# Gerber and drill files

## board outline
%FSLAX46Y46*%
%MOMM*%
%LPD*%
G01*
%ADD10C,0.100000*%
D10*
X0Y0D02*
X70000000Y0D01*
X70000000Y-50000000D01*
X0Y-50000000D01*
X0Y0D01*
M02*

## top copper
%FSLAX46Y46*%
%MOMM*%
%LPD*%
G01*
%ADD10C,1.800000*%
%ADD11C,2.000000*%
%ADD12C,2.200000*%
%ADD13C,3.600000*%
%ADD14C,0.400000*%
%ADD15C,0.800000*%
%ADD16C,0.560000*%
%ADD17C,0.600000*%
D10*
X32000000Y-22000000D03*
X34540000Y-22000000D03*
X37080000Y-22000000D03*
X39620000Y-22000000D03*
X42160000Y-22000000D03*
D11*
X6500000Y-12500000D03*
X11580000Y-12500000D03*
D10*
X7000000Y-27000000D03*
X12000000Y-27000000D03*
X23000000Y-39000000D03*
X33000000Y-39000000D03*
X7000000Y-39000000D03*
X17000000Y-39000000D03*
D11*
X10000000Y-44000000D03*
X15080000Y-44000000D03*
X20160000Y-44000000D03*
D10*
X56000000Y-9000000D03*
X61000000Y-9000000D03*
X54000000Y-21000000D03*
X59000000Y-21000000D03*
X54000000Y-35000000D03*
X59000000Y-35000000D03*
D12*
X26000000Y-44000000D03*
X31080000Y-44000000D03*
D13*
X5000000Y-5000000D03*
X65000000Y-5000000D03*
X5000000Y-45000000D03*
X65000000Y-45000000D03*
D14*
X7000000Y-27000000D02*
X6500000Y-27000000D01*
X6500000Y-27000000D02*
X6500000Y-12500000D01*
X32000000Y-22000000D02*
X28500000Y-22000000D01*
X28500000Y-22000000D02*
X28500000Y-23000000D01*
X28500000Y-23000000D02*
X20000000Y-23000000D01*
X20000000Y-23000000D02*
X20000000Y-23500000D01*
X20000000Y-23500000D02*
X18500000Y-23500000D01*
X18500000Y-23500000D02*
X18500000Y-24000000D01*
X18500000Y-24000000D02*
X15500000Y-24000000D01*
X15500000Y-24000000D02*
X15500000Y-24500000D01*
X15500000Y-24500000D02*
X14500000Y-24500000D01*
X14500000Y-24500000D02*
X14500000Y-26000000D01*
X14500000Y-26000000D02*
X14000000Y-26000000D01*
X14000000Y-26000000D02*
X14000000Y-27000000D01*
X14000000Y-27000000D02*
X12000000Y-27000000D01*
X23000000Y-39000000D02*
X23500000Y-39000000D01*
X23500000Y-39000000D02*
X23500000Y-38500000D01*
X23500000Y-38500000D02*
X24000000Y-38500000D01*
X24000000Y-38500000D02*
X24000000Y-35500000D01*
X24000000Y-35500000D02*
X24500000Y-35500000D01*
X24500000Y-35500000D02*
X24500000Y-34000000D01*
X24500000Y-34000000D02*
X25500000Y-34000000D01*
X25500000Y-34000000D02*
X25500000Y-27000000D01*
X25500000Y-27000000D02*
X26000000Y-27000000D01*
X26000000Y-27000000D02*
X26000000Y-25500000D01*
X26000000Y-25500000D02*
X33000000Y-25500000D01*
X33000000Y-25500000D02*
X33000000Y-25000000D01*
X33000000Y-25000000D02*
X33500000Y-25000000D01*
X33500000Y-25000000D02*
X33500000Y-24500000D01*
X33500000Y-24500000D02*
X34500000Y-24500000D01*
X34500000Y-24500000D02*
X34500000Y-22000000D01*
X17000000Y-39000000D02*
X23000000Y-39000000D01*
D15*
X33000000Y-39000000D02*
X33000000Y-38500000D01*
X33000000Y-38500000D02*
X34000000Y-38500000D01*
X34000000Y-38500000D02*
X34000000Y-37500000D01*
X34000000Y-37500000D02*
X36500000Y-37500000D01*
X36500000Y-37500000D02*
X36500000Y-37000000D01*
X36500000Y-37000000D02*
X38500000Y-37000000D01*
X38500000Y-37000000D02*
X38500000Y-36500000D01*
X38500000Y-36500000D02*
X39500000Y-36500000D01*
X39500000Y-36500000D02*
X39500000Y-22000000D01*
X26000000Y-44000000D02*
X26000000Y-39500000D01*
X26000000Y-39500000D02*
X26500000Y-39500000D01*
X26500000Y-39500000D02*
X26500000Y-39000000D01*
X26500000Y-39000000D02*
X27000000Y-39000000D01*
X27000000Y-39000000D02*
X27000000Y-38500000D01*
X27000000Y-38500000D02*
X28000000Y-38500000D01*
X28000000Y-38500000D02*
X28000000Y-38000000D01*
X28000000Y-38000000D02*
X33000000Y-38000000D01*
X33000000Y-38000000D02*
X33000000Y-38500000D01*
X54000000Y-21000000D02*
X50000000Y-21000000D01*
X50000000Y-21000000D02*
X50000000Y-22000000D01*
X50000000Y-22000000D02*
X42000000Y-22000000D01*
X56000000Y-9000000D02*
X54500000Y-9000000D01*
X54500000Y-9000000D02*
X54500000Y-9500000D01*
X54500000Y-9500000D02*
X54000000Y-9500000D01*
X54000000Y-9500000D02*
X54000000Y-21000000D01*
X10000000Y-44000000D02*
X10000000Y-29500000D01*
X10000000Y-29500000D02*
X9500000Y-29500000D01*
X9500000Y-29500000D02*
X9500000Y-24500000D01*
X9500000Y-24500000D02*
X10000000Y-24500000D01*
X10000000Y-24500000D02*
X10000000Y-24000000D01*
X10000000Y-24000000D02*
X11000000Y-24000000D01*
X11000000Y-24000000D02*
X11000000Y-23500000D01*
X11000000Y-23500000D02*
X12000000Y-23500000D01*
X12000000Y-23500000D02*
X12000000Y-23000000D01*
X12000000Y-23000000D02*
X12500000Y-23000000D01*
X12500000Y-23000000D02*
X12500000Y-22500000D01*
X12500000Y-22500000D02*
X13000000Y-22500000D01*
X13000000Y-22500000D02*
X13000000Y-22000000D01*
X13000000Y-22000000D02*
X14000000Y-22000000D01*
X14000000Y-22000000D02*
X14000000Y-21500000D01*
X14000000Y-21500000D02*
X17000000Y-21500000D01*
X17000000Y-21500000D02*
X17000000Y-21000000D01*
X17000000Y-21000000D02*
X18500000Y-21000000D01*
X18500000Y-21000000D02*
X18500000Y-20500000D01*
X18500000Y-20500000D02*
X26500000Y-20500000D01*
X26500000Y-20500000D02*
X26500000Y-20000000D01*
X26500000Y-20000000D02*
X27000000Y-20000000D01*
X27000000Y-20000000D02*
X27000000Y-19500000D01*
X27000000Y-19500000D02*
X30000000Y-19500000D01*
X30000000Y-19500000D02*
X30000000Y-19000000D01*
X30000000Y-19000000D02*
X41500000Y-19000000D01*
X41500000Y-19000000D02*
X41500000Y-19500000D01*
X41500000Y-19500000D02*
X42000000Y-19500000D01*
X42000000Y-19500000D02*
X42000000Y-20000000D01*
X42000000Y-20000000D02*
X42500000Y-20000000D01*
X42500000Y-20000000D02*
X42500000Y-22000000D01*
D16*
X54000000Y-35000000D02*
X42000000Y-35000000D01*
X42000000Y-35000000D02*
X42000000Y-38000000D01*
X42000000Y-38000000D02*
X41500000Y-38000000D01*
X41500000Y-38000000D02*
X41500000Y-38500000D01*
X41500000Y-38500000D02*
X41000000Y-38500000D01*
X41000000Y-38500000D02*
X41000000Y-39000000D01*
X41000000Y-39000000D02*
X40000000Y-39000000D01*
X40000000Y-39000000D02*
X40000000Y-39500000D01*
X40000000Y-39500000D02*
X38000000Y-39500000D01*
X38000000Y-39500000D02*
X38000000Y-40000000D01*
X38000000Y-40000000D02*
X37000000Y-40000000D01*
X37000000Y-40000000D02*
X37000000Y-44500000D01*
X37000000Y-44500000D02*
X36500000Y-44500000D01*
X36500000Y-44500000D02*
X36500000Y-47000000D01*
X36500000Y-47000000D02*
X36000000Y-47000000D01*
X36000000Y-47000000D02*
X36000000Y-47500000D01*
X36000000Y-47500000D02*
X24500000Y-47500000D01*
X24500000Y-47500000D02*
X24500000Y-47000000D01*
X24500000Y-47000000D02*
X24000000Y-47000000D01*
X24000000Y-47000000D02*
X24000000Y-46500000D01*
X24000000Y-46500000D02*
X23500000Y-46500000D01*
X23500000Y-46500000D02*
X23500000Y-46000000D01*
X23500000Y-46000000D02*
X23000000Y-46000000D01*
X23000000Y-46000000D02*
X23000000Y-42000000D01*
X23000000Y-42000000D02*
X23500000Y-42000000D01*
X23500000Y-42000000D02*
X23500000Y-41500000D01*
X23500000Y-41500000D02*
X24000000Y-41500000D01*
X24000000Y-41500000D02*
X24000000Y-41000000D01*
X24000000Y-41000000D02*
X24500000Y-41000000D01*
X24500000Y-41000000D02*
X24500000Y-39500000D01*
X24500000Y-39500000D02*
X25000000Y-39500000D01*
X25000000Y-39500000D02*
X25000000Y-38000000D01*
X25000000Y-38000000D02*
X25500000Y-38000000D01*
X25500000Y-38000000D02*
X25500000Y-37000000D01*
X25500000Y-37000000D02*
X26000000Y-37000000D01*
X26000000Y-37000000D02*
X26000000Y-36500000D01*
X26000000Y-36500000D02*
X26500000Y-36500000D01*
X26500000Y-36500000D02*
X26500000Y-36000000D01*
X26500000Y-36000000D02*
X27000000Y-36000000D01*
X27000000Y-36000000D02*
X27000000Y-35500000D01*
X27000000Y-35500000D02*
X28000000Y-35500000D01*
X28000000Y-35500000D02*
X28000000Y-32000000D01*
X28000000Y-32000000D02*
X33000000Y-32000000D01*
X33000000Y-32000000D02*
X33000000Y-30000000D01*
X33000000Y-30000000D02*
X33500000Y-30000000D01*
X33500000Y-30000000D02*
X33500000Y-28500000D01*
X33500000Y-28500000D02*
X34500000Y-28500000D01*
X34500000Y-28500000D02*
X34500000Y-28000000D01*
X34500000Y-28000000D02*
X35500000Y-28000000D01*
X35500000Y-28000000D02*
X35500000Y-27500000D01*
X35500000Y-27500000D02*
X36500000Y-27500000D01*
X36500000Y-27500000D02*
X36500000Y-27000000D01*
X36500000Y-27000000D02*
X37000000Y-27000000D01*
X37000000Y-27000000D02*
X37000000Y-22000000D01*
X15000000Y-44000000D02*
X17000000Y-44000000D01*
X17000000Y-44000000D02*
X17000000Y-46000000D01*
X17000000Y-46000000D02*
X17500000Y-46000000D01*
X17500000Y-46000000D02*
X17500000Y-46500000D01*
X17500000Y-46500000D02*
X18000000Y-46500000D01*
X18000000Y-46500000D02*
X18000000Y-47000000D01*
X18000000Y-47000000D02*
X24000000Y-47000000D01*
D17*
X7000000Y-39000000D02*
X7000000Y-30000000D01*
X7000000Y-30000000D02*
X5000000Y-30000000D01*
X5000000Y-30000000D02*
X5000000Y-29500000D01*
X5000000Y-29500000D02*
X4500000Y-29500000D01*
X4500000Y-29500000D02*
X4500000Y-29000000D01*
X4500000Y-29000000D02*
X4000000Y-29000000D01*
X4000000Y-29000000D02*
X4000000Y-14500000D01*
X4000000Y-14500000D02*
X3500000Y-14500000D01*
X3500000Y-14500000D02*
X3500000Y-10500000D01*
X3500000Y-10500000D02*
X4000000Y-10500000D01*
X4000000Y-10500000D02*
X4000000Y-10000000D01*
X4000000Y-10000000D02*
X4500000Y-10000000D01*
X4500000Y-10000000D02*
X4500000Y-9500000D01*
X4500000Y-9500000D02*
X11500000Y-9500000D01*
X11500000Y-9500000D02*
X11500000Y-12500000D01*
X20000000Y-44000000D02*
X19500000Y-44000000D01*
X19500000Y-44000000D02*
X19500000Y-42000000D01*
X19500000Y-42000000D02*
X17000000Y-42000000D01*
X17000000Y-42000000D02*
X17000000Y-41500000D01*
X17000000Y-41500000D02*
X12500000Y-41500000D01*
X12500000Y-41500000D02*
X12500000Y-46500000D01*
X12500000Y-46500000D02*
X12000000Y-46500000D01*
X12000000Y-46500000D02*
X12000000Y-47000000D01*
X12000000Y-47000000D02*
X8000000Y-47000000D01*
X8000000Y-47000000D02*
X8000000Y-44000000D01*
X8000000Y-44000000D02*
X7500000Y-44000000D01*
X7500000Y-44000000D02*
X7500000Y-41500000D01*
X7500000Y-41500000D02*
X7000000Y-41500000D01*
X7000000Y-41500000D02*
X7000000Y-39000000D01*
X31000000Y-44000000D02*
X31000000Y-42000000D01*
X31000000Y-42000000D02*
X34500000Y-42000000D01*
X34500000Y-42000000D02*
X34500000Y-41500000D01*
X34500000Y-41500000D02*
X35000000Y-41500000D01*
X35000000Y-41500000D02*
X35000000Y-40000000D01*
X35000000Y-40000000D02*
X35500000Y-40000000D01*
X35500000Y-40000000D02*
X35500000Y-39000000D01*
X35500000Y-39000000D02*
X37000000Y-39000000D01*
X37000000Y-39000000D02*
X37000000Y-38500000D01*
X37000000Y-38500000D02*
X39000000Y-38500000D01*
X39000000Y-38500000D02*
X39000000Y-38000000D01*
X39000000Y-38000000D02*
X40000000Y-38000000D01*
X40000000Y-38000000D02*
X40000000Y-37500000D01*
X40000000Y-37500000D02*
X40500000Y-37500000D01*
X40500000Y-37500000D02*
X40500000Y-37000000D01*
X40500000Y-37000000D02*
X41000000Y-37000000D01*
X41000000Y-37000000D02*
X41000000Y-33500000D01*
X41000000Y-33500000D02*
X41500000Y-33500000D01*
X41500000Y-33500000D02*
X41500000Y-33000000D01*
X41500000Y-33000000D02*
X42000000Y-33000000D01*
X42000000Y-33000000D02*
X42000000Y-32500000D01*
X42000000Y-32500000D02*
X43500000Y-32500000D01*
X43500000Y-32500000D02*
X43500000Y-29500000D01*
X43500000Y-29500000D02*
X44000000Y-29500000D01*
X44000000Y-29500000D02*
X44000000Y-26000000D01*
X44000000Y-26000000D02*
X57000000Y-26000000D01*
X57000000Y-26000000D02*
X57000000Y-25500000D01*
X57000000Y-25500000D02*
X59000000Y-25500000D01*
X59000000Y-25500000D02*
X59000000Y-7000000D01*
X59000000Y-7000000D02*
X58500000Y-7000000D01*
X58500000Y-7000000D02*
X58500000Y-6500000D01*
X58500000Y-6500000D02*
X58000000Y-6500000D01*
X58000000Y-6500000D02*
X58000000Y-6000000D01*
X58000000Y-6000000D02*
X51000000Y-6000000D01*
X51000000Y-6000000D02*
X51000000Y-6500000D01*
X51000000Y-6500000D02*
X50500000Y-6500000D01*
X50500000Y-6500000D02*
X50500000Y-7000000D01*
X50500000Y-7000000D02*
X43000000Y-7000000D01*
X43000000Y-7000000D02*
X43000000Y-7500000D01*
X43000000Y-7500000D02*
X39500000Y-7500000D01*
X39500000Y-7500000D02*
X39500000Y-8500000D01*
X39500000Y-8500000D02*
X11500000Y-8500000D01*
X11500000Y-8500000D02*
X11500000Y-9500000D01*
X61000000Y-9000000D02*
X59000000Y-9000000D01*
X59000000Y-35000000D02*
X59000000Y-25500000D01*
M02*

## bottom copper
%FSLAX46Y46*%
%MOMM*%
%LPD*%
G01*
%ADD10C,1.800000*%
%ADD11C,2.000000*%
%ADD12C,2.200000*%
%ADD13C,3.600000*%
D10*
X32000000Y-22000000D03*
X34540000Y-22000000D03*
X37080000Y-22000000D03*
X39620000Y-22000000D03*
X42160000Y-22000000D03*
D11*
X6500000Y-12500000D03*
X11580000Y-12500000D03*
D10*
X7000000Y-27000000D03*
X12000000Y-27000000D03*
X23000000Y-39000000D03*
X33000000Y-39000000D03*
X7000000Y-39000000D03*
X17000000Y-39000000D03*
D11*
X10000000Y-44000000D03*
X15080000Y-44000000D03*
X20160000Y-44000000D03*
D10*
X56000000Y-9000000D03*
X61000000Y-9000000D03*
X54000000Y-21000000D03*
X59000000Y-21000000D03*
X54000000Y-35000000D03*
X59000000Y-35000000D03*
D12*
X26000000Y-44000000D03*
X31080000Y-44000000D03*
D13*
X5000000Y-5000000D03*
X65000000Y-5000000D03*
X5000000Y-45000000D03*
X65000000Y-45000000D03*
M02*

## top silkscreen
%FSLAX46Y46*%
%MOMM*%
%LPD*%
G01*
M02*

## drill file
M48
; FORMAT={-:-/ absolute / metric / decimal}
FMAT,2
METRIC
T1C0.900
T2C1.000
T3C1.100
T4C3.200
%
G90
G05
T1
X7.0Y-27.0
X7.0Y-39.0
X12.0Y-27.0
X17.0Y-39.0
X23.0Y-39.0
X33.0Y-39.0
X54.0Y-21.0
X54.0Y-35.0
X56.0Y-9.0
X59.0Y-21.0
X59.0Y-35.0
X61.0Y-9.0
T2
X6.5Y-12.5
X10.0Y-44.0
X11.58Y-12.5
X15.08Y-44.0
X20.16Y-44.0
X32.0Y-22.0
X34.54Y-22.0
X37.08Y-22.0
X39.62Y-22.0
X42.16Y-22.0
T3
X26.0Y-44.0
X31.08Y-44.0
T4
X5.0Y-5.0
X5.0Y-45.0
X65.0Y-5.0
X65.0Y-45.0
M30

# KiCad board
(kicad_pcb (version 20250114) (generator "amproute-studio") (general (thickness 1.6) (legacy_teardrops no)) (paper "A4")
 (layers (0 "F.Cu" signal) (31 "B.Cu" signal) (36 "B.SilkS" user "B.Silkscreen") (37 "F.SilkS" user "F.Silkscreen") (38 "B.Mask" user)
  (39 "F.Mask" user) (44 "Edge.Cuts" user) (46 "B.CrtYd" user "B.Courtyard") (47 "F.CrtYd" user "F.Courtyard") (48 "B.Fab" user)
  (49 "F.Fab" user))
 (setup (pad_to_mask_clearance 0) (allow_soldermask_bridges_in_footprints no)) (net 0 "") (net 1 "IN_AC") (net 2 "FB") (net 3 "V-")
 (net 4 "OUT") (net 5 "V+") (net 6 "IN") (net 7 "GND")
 (gr_rect (start 0 0) (end 70.0000 50.0000) (stroke (width 0.1) (type default)) (fill none) (layer "Edge.Cuts"))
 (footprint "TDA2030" (layer "F.Cu") (at 30.0000 14.0000)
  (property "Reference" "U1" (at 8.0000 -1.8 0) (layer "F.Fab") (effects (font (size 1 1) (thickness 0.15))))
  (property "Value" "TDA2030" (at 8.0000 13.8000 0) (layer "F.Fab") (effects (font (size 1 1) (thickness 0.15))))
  (pad "1" thru_hole circle (at 2.0000 8.0000) (size 1.8000 1.8000) (drill 1.0000) (layers "*.Cu" "*.Mask") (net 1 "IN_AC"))
  (pad "2" thru_hole circle (at 4.5400 8.0000) (size 1.8000 1.8000) (drill 1.0000) (layers "*.Cu" "*.Mask") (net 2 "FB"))
  (pad "3" thru_hole circle (at 7.0800 8.0000) (size 1.8000 1.8000) (drill 1.0000) (layers "*.Cu" "*.Mask") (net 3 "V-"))
  (pad "4" thru_hole circle (at 9.6200 8.0000) (size 1.8000 1.8000) (drill 1.0000) (layers "*.Cu" "*.Mask") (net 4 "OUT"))
  (pad "5" thru_hole circle (at 12.1600 8.0000) (size 1.8000 1.8000) (drill 1.0000) (layers "*.Cu" "*.Mask") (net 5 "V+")))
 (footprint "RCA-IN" (layer "F.Cu") (at 4.0000 8.0000)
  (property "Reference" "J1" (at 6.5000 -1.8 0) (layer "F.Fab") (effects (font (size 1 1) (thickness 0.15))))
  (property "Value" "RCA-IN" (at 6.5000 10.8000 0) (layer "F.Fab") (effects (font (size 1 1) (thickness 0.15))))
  (pad "1" thru_hole circle (at 2.5000 4.5000) (size 2.0000 2.0000) (drill 1.0000) (layers "*.Cu" "*.Mask") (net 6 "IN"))
  (pad "2" thru_hole circle (at 7.5800 4.5000) (size 2.0000 2.0000) (drill 1.0000) (layers "*.Cu" "*.Mask") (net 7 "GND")))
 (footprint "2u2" (layer "F.Cu") (at 5.0000 24.0000)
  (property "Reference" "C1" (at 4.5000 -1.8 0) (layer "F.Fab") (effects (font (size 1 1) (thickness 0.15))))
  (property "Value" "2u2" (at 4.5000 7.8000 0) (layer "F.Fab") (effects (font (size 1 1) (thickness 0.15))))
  (pad "1" thru_hole circle (at 2.0000 3.0000) (size 1.8000 1.8000) (drill 0.9000) (layers "*.Cu" "*.Mask") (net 6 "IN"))
  (pad "2" thru_hole circle (at 7.0000 3.0000) (size 1.8000 1.8000) (drill 0.9000) (layers "*.Cu" "*.Mask") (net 1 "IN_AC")))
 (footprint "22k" (layer "F.Cu") (at 22.0000 36.0000)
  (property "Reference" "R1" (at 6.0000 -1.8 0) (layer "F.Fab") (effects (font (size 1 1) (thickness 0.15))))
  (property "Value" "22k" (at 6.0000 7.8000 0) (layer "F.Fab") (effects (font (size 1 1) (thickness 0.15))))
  (pad "1" thru_hole circle (at 1.0000 3.0000) (size 1.8000 1.8000) (drill 0.9000) (layers "*.Cu" "*.Mask") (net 2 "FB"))
  (pad "2" thru_hole circle (at 11.0000 3.0000) (size 1.8000 1.8000) (drill 0.9000) (layers "*.Cu" "*.Mask") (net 4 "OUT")))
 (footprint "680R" (layer "F.Cu") (at 6.0000 36.0000)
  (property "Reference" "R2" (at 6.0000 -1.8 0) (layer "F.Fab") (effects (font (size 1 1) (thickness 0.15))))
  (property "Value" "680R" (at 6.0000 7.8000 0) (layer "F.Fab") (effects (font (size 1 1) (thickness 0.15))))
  (pad "1" thru_hole circle (at 1.0000 3.0000) (size 1.8000 1.8000) (drill 0.9000) (layers "*.Cu" "*.Mask") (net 7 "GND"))
  (pad "2" thru_hole circle (at 11.0000 3.0000) (size 1.8000 1.8000) (drill 0.9000) (layers "*.Cu" "*.Mask") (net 2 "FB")))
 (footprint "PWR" (layer "F.Cu") (at 8.0000 40.0000)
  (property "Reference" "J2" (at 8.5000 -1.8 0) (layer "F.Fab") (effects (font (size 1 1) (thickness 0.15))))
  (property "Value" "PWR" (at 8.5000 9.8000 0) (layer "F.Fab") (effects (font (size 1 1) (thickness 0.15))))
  (pad "1" thru_hole circle (at 2.0000 4.0000) (size 2.0000 2.0000) (drill 1.0000) (layers "*.Cu" "*.Mask") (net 5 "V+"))
  (pad "2" thru_hole circle (at 7.0800 4.0000) (size 2.0000 2.0000) (drill 1.0000) (layers "*.Cu" "*.Mask") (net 3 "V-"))
  (pad "3" thru_hole circle (at 12.1600 4.0000) (size 2.0000 2.0000) (drill 1.0000) (layers "*.Cu" "*.Mask") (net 7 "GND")))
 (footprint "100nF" (layer "F.Cu") (at 54.0000 6.0000)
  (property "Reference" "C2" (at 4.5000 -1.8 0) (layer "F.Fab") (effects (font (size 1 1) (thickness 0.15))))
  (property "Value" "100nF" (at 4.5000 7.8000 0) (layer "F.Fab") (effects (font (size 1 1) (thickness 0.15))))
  (pad "1" thru_hole circle (at 2.0000 3.0000) (size 1.8000 1.8000) (drill 0.9000) (layers "*.Cu" "*.Mask") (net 5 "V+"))
  (pad "2" thru_hole circle (at 7.0000 3.0000) (size 1.8000 1.8000) (drill 0.9000) (layers "*.Cu" "*.Mask") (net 7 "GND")))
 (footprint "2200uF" (layer "F.Cu") (at 52.0000 18.0000)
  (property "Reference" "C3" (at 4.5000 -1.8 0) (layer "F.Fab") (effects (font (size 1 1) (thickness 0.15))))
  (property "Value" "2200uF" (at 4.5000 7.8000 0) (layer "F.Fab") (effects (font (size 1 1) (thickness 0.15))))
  (pad "1" thru_hole circle (at 2.0000 3.0000) (size 1.8000 1.8000) (drill 0.9000) (layers "*.Cu" "*.Mask") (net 5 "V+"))
  (pad "2" thru_hole circle (at 7.0000 3.0000) (size 1.8000 1.8000) (drill 0.9000) (layers "*.Cu" "*.Mask") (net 7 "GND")))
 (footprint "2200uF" (layer "F.Cu") (at 52.0000 32.0000)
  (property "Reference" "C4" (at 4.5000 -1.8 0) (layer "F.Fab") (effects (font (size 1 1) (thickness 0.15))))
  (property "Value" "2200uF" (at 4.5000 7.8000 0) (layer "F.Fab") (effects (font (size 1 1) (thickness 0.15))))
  (pad "1" thru_hole circle (at 2.0000 3.0000) (size 1.8000 1.8000) (drill 0.9000) (layers "*.Cu" "*.Mask") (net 3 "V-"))
  (pad "2" thru_hole circle (at 7.0000 3.0000) (size 1.8000 1.8000) (drill 0.9000) (layers "*.Cu" "*.Mask") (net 7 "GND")))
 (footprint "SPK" (layer "F.Cu") (at 24.0000 40.0000)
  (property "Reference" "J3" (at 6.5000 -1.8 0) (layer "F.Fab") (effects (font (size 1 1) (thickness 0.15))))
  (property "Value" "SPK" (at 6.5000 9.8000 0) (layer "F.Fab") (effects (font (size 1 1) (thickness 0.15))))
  (pad "1" thru_hole circle (at 2.0000 4.0000) (size 2.2000 2.2000) (drill 1.1000) (layers "*.Cu" "*.Mask") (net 4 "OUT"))
  (pad "2" thru_hole circle (at 7.0800 4.0000) (size 2.2000 2.2000) (drill 1.1000) (layers "*.Cu" "*.Mask") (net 7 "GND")))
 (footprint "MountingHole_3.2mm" (layer "F.Cu") (at 5.0000 5.0000)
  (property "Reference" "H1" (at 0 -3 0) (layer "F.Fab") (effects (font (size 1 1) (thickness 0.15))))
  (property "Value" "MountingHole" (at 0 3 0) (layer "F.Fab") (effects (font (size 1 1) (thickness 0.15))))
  (pad "" np_thru_hole circle (at 0 0) (size 3.6000 3.6000) (drill 3.2000) (layers "*.Cu" "*.Mask")))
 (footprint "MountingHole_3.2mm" (layer "F.Cu") (at 65.0000 5.0000)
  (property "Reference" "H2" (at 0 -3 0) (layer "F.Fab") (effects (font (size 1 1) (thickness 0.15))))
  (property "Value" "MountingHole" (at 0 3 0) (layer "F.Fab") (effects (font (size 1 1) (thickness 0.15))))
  (pad "" np_thru_hole circle (at 0 0) (size 3.6000 3.6000) (drill 3.2000) (layers "*.Cu" "*.Mask")))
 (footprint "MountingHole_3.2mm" (layer "F.Cu") (at 5.0000 45.0000)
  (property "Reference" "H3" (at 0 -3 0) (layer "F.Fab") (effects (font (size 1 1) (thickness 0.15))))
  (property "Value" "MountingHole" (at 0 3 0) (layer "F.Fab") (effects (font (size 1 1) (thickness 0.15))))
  (pad "" np_thru_hole circle (at 0 0) (size 3.6000 3.6000) (drill 3.2000) (layers "*.Cu" "*.Mask")))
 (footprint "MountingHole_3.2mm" (layer "F.Cu") (at 65.0000 45.0000)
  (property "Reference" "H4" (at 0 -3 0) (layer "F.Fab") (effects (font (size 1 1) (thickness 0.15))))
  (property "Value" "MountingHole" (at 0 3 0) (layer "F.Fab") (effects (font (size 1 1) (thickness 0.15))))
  (pad "" np_thru_hole circle (at 0 0) (size 3.6000 3.6000) (drill 3.2000) (layers "*.Cu" "*.Mask")))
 (segment (start 7.0000 27.0000) (end 6.5000 27.0000) (width 0.4000) (layer "F.Cu") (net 6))
 (segment (start 6.5000 27.0000) (end 6.5000 12.5000) (width 0.4000) (layer "F.Cu") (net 6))
 (segment (start 32.0000 22.0000) (end 28.5000 22.0000) (width 0.4000) (layer "F.Cu") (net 1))
 (segment (start 28.5000 22.0000) (end 28.5000 23.0000) (width 0.4000) (layer "F.Cu") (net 1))
 (segment (start 28.5000 23.0000) (end 20.0000 23.0000) (width 0.4000) (layer "F.Cu") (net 1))
 (segment (start 20.0000 23.0000) (end 20.0000 23.5000) (width 0.4000) (layer "F.Cu") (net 1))
 (segment (start 20.0000 23.5000) (end 18.5000 23.5000) (width 0.4000) (layer "F.Cu") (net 1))
 (segment (start 18.5000 23.5000) (end 18.5000 24.0000) (width 0.4000) (layer "F.Cu") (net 1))
 (segment (start 18.5000 24.0000) (end 15.5000 24.0000) (width 0.4000) (layer "F.Cu") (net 1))
 (segment (start 15.5000 24.0000) (end 15.5000 24.5000) (width 0.4000) (layer "F.Cu") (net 1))
 (segment (start 15.5000 24.5000) (end 14.5000 24.5000) (width 0.4000) (layer "F.Cu") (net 1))
 (segment (start 14.5000 24.5000) (end 14.5000 26.0000) (width 0.4000) (layer "F.Cu") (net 1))
 (segment (start 14.5000 26.0000) (end 14.0000 26.0000) (width 0.4000) (layer "F.Cu") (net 1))
 (segment (start 14.0000 26.0000) (end 14.0000 27.0000) (width 0.4000) (layer "F.Cu") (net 1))
 (segment (start 14.0000 27.0000) (end 12.0000 27.0000) (width 0.4000) (layer "F.Cu") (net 1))
 (segment (start 23.0000 39.0000) (end 23.5000 39.0000) (width 0.4000) (layer "F.Cu") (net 2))
 (segment (start 23.5000 39.0000) (end 23.5000 38.5000) (width 0.4000) (layer "F.Cu") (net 2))
 (segment (start 23.5000 38.5000) (end 24.0000 38.5000) (width 0.4000) (layer "F.Cu") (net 2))
 (segment (start 24.0000 38.5000) (end 24.0000 35.5000) (width 0.4000) (layer "F.Cu") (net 2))
 (segment (start 24.0000 35.5000) (end 24.5000 35.5000) (width 0.4000) (layer "F.Cu") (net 2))
 (segment (start 24.5000 35.5000) (end 24.5000 34.0000) (width 0.4000) (layer "F.Cu") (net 2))
 (segment (start 24.5000 34.0000) (end 25.5000 34.0000) (width 0.4000) (layer "F.Cu") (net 2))
 (segment (start 25.5000 34.0000) (end 25.5000 27.0000) (width 0.4000) (layer "F.Cu") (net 2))
 (segment (start 25.5000 27.0000) (end 26.0000 27.0000) (width 0.4000) (layer "F.Cu") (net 2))
 (segment (start 26.0000 27.0000) (end 26.0000 25.5000) (width 0.4000) (layer "F.Cu") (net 2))
 (segment (start 26.0000 25.5000) (end 33.0000 25.5000) (width 0.4000) (layer "F.Cu") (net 2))
 (segment (start 33.0000 25.5000) (end 33.0000 25.0000) (width 0.4000) (layer "F.Cu") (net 2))
 (segment (start 33.0000 25.0000) (end 33.5000 25.0000) (width 0.4000) (layer "F.Cu") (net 2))
 (segment (start 33.5000 25.0000) (end 33.5000 24.5000) (width 0.4000) (layer "F.Cu") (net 2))
 (segment (start 33.5000 24.5000) (end 34.5000 24.5000) (width 0.4000) (layer "F.Cu") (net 2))
 (segment (start 34.5000 24.5000) (end 34.5000 22.0000) (width 0.4000) (layer "F.Cu") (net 2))
 (segment (start 17.0000 39.0000) (end 23.0000 39.0000) (width 0.4000) (layer "F.Cu") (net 2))
 (segment (start 33.0000 39.0000) (end 33.0000 38.5000) (width 0.8000) (layer "F.Cu") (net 4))
 (segment (start 33.0000 38.5000) (end 34.0000 38.5000) (width 0.8000) (layer "F.Cu") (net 4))
 (segment (start 34.0000 38.5000) (end 34.0000 37.5000) (width 0.8000) (layer "F.Cu") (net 4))
 (segment (start 34.0000 37.5000) (end 36.5000 37.5000) (width 0.8000) (layer "F.Cu") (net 4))
 (segment (start 36.5000 37.5000) (end 36.5000 37.0000) (width 0.8000) (layer "F.Cu") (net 4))
 (segment (start 36.5000 37.0000) (end 38.5000 37.0000) (width 0.8000) (layer "F.Cu") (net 4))
 (segment (start 38.5000 37.0000) (end 38.5000 36.5000) (width 0.8000) (layer "F.Cu") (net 4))
 (segment (start 38.5000 36.5000) (end 39.5000 36.5000) (width 0.8000) (layer "F.Cu") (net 4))
 (segment (start 39.5000 36.5000) (end 39.5000 22.0000) (width 0.8000) (layer "F.Cu") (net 4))
 (segment (start 26.0000 44.0000) (end 26.0000 39.5000) (width 0.8000) (layer "F.Cu") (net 4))
 (segment (start 26.0000 39.5000) (end 26.5000 39.5000) (width 0.8000) (layer "F.Cu") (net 4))
 (segment (start 26.5000 39.5000) (end 26.5000 39.0000) (width 0.8000) (layer "F.Cu") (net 4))
 (segment (start 26.5000 39.0000) (end 27.0000 39.0000) (width 0.8000) (layer "F.Cu") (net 4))
 (segment (start 27.0000 39.0000) (end 27.0000 38.5000) (width 0.8000) (layer "F.Cu") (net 4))
 (segment (start 27.0000 38.5000) (end 28.0000 38.5000) (width 0.8000) (layer "F.Cu") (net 4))
 (segment (start 28.0000 38.5000) (end 28.0000 38.0000) (width 0.8000) (layer "F.Cu") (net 4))
 (segment (start 28.0000 38.0000) (end 33.0000 38.0000) (width 0.8000) (layer "F.Cu") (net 4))
 (segment (start 33.0000 38.0000) (end 33.0000 38.5000) (width 0.8000) (layer "F.Cu") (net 4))
 (segment (start 54.0000 21.0000) (end 50.0000 21.0000) (width 0.8000) (layer "F.Cu") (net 5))
 (segment (start 50.0000 21.0000) (end 50.0000 22.0000) (width 0.8000) (layer "F.Cu") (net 5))
 (segment (start 50.0000 22.0000) (end 42.0000 22.0000) (width 0.8000) (layer "F.Cu") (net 5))
 (segment (start 56.0000 9.0000) (end 54.5000 9.0000) (width 0.8000) (layer "F.Cu") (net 5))
 (segment (start 54.5000 9.0000) (end 54.5000 9.5000) (width 0.8000) (layer "F.Cu") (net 5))
 (segment (start 54.5000 9.5000) (end 54.0000 9.5000) (width 0.8000) (layer "F.Cu") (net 5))
 (segment (start 54.0000 9.5000) (end 54.0000 21.0000) (width 0.8000) (layer "F.Cu") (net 5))
 (segment (start 10.0000 44.0000) (end 10.0000 29.5000) (width 0.8000) (layer "F.Cu") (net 5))
 (segment (start 10.0000 29.5000) (end 9.5000 29.5000) (width 0.8000) (layer "F.Cu") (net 5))
 (segment (start 9.5000 29.5000) (end 9.5000 24.5000) (width 0.8000) (layer "F.Cu") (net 5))
 (segment (start 9.5000 24.5000) (end 10.0000 24.5000) (width 0.8000) (layer "F.Cu") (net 5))
 (segment (start 10.0000 24.5000) (end 10.0000 24.0000) (width 0.8000) (layer "F.Cu") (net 5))
 (segment (start 10.0000 24.0000) (end 11.0000 24.0000) (width 0.8000) (layer "F.Cu") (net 5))
 (segment (start 11.0000 24.0000) (end 11.0000 23.5000) (width 0.8000) (layer "F.Cu") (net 5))
 (segment (start 11.0000 23.5000) (end 12.0000 23.5000) (width 0.8000) (layer "F.Cu") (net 5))
 (segment (start 12.0000 23.5000) (end 12.0000 23.0000) (width 0.8000) (layer "F.Cu") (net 5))
 (segment (start 12.0000 23.0000) (end 12.5000 23.0000) (width 0.8000) (layer "F.Cu") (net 5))
 (segment (start 12.5000 23.0000) (end 12.5000 22.5000) (width 0.8000) (layer "F.Cu") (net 5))
 (segment (start 12.5000 22.5000) (end 13.0000 22.5000) (width 0.8000) (layer "F.Cu") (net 5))
 (segment (start 13.0000 22.5000) (end 13.0000 22.0000) (width 0.8000) (layer "F.Cu") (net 5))
 (segment (start 13.0000 22.0000) (end 14.0000 22.0000) (width 0.8000) (layer "F.Cu") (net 5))
 (segment (start 14.0000 22.0000) (end 14.0000 21.5000) (width 0.8000) (layer "F.Cu") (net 5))
 (segment (start 14.0000 21.5000) (end 17.0000 21.5000) (width 0.8000) (layer "F.Cu") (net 5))
 (segment (start 17.0000 21.5000) (end 17.0000 21.0000) (width 0.8000) (layer "F.Cu") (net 5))
 (segment (start 17.0000 21.0000) (end 18.5000 21.0000) (width 0.8000) (layer "F.Cu") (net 5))
 (segment (start 18.5000 21.0000) (end 18.5000 20.5000) (width 0.8000) (layer "F.Cu") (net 5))
 (segment (start 18.5000 20.5000) (end 26.5000 20.5000) (width 0.8000) (layer "F.Cu") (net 5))
 (segment (start 26.5000 20.5000) (end 26.5000 20.0000) (width 0.8000) (layer "F.Cu") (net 5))
 (segment (start 26.5000 20.0000) (end 27.0000 20.0000) (width 0.8000) (layer "F.Cu") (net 5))
 (segment (start 27.0000 20.0000) (end 27.0000 19.5000) (width 0.8000) (layer "F.Cu") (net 5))
 (segment (start 27.0000 19.5000) (end 30.0000 19.5000) (width 0.8000) (layer "F.Cu") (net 5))
 (segment (start 30.0000 19.5000) (end 30.0000 19.0000) (width 0.8000) (layer "F.Cu") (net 5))
 (segment (start 30.0000 19.0000) (end 41.5000 19.0000) (width 0.8000) (layer "F.Cu") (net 5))
 (segment (start 41.5000 19.0000) (end 41.5000 19.5000) (width 0.8000) (layer "F.Cu") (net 5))
 (segment (start 41.5000 19.5000) (end 42.0000 19.5000) (width 0.8000) (layer "F.Cu") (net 5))
 (segment (start 42.0000 19.5000) (end 42.0000 20.0000) (width 0.8000) (layer "F.Cu") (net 5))
 (segment (start 42.0000 20.0000) (end 42.5000 20.0000) (width 0.8000) (layer "F.Cu") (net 5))
 (segment (start 42.5000 20.0000) (end 42.5000 22.0000) (width 0.8000) (layer "F.Cu") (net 5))
 (segment (start 54.0000 35.0000) (end 42.0000 35.0000) (width 0.5600) (layer "F.Cu") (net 3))
 (segment (start 42.0000 35.0000) (end 42.0000 38.0000) (width 0.5600) (layer "F.Cu") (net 3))
 (segment (start 42.0000 38.0000) (end 41.5000 38.0000) (width 0.5600) (layer "F.Cu") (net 3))
 (segment (start 41.5000 38.0000) (end 41.5000 38.5000) (width 0.5600) (layer "F.Cu") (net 3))
 (segment (start 41.5000 38.5000) (end 41.0000 38.5000) (width 0.5600) (layer "F.Cu") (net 3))
 (segment (start 41.0000 38.5000) (end 41.0000 39.0000) (width 0.5600) (layer "F.Cu") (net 3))
 (segment (start 41.0000 39.0000) (end 40.0000 39.0000) (width 0.5600) (layer "F.Cu") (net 3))
 (segment (start 40.0000 39.0000) (end 40.0000 39.5000) (width 0.5600) (layer "F.Cu") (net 3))
 (segment (start 40.0000 39.5000) (end 38.0000 39.5000) (width 0.5600) (layer "F.Cu") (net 3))
 (segment (start 38.0000 39.5000) (end 38.0000 40.0000) (width 0.5600) (layer "F.Cu") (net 3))
 (segment (start 38.0000 40.0000) (end 37.0000 40.0000) (width 0.5600) (layer "F.Cu") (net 3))
 (segment (start 37.0000 40.0000) (end 37.0000 44.5000) (width 0.5600) (layer "F.Cu") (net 3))
 (segment (start 37.0000 44.5000) (end 36.5000 44.5000) (width 0.5600) (layer "F.Cu") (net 3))
 (segment (start 36.5000 44.5000) (end 36.5000 47.0000) (width 0.5600) (layer "F.Cu") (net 3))
 (segment (start 36.5000 47.0000) (end 36.0000 47.0000) (width 0.5600) (layer "F.Cu") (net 3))
 (segment (start 36.0000 47.0000) (end 36.0000 47.5000) (width 0.5600) (layer "F.Cu") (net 3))
 (segment (start 36.0000 47.5000) (end 24.5000 47.5000) (width 0.5600) (layer "F.Cu") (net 3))
 (segment (start 24.5000 47.5000) (end 24.5000 47.0000) (width 0.5600) (layer "F.Cu") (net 3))
 (segment (start 24.5000 47.0000) (end 24.0000 47.0000) (width 0.5600) (layer "F.Cu") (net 3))
 (segment (start 24.0000 47.0000) (end 24.0000 46.5000) (width 0.5600) (layer "F.Cu") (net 3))
 (segment (start 24.0000 46.5000) (end 23.5000 46.5000) (width 0.5600) (layer "F.Cu") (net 3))
 (segment (start 23.5000 46.5000) (end 23.5000 46.0000) (width 0.5600) (layer "F.Cu") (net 3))
 (segment (start 23.5000 46.0000) (end 23.0000 46.0000) (width 0.5600) (layer "F.Cu") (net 3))
 (segment (start 23.0000 46.0000) (end 23.0000 42.0000) (width 0.5600) (layer "F.Cu") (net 3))
 (segment (start 23.0000 42.0000) (end 23.5000 42.0000) (width 0.5600) (layer "F.Cu") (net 3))
 (segment (start 23.5000 42.0000) (end 23.5000 41.5000) (width 0.5600) (layer "F.Cu") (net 3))
 (segment (start 23.5000 41.5000) (end 24.0000 41.5000) (width 0.5600) (layer "F.Cu") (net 3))
 (segment (start 24.0000 41.5000) (end 24.0000 41.0000) (width 0.5600) (layer "F.Cu") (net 3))
 (segment (start 24.0000 41.0000) (end 24.5000 41.0000) (width 0.5600) (layer "F.Cu") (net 3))
 (segment (start 24.5000 41.0000) (end 24.5000 39.5000) (width 0.5600) (layer "F.Cu") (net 3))
 (segment (start 24.5000 39.5000) (end 25.0000 39.5000) (width 0.5600) (layer "F.Cu") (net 3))
 (segment (start 25.0000 39.5000) (end 25.0000 38.0000) (width 0.5600) (layer "F.Cu") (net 3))
 (segment (start 25.0000 38.0000) (end 25.5000 38.0000) (width 0.5600) (layer "F.Cu") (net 3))
 (segment (start 25.5000 38.0000) (end 25.5000 37.0000) (width 0.5600) (layer "F.Cu") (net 3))
 (segment (start 25.5000 37.0000) (end 26.0000 37.0000) (width 0.5600) (layer "F.Cu") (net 3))
 (segment (start 26.0000 37.0000) (end 26.0000 36.5000) (width 0.5600) (layer "F.Cu") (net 3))
 (segment (start 26.0000 36.5000) (end 26.5000 36.5000) (width 0.5600) (layer "F.Cu") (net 3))
 (segment (start 26.5000 36.5000) (end 26.5000 36.0000) (width 0.5600) (layer "F.Cu") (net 3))
 (segment (start 26.5000 36.0000) (end 27.0000 36.0000) (width 0.5600) (layer "F.Cu") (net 3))
 (segment (start 27.0000 36.0000) (end 27.0000 35.5000) (width 0.5600) (layer "F.Cu") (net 3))
 (segment (start 27.0000 35.5000) (end 28.0000 35.5000) (width 0.5600) (layer "F.Cu") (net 3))
 (segment (start 28.0000 35.5000) (end 28.0000 32.0000) (width 0.5600) (layer "F.Cu") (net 3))
 (segment (start 28.0000 32.0000) (end 33.0000 32.0000) (width 0.5600) (layer "F.Cu") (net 3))
 (segment (start 33.0000 32.0000) (end 33.0000 30.0000) (width 0.5600) (layer "F.Cu") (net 3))
 (segment (start 33.0000 30.0000) (end 33.5000 30.0000) (width 0.5600) (layer "F.Cu") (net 3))
 (segment (start 33.5000 30.0000) (end 33.5000 28.5000) (width 0.5600) (layer "F.Cu") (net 3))
 (segment (start 33.5000 28.5000) (end 34.5000 28.5000) (width 0.5600) (layer "F.Cu") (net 3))
 (segment (start 34.5000 28.5000) (end 34.5000 28.0000) (width 0.5600) (layer "F.Cu") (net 3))
 (segment (start 34.5000 28.0000) (end 35.5000 28.0000) (width 0.5600) (layer "F.Cu") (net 3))
 (segment (start 35.5000 28.0000) (end 35.5000 27.5000) (width 0.5600) (layer "F.Cu") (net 3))
 (segment (start 35.5000 27.5000) (end 36.5000 27.5000) (width 0.5600) (layer "F.Cu") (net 3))
 (segment (start 36.5000 27.5000) (end 36.5000 27.0000) (width 0.5600) (layer "F.Cu") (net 3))
 (segment (start 36.5000 27.0000) (end 37.0000 27.0000) (width 0.5600) (layer "F.Cu") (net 3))
 (segment (start 37.0000 27.0000) (end 37.0000 22.0000) (width 0.5600) (layer "F.Cu") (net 3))
 (segment (start 15.0000 44.0000) (end 17.0000 44.0000) (width 0.5600) (layer "F.Cu") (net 3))
 (segment (start 17.0000 44.0000) (end 17.0000 46.0000) (width 0.5600) (layer "F.Cu") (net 3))
 (segment (start 17.0000 46.0000) (end 17.5000 46.0000) (width 0.5600) (layer "F.Cu") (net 3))
 (segment (start 17.5000 46.0000) (end 17.5000 46.5000) (width 0.5600) (layer "F.Cu") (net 3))
 (segment (start 17.5000 46.5000) (end 18.0000 46.5000) (width 0.5600) (layer "F.Cu") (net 3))
 (segment (start 18.0000 46.5000) (end 18.0000 47.0000) (width 0.5600) (layer "F.Cu") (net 3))
 (segment (start 18.0000 47.0000) (end 24.0000 47.0000) (width 0.5600) (layer "F.Cu") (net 3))
 (segment (start 7.0000 39.0000) (end 7.0000 30.0000) (width 0.6000) (layer "F.Cu") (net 7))
 (segment (start 7.0000 30.0000) (end 5.0000 30.0000) (width 0.6000) (layer "F.Cu") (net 7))
 (segment (start 5.0000 30.0000) (end 5.0000 29.5000) (width 0.6000) (layer "F.Cu") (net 7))
 (segment (start 5.0000 29.5000) (end 4.5000 29.5000) (width 0.6000) (layer "F.Cu") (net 7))
 (segment (start 4.5000 29.5000) (end 4.5000 29.0000) (width 0.6000) (layer "F.Cu") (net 7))
 (segment (start 4.5000 29.0000) (end 4.0000 29.0000) (width 0.6000) (layer "F.Cu") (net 7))
 (segment (start 4.0000 29.0000) (end 4.0000 14.5000) (width 0.6000) (layer "F.Cu") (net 7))
 (segment (start 4.0000 14.5000) (end 3.5000 14.5000) (width 0.6000) (layer "F.Cu") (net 7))
 (segment (start 3.5000 14.5000) (end 3.5000 10.5000) (width 0.6000) (layer "F.Cu") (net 7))
 (segment (start 3.5000 10.5000) (end 4.0000 10.5000) (width 0.6000) (layer "F.Cu") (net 7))
 (segment (start 4.0000 10.5000) (end 4.0000 10.0000) (width 0.6000) (layer "F.Cu") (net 7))
 (segment (start 4.0000 10.0000) (end 4.5000 10.0000) (width 0.6000) (layer "F.Cu") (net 7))
 (segment (start 4.5000 10.0000) (end 4.5000 9.5000) (width 0.6000) (layer "F.Cu") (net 7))
 (segment (start 4.5000 9.5000) (end 11.5000 9.5000) (width 0.6000) (layer "F.Cu") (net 7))
 (segment (start 11.5000 9.5000) (end 11.5000 12.5000) (width 0.6000) (layer "F.Cu") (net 7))
 (segment (start 20.0000 44.0000) (end 19.5000 44.0000) (width 0.6000) (layer "F.Cu") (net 7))
 (segment (start 19.5000 44.0000) (end 19.5000 42.0000) (width 0.6000) (layer "F.Cu") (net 7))
 (segment (start 19.5000 42.0000) (end 17.0000 42.0000) (width 0.6000) (layer "F.Cu") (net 7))
 (segment (start 17.0000 42.0000) (end 17.0000 41.5000) (width 0.6000) (layer "F.Cu") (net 7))
 (segment (start 17.0000 41.5000) (end 12.5000 41.5000) (width 0.6000) (layer "F.Cu") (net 7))
 (segment (start 12.5000 41.5000) (end 12.5000 46.5000) (width 0.6000) (layer "F.Cu") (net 7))
 (segment (start 12.5000 46.5000) (end 12.0000 46.5000) (width 0.6000) (layer "F.Cu") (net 7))
 (segment (start 12.0000 46.5000) (end 12.0000 47.0000) (width 0.6000) (layer "F.Cu") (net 7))
 (segment (start 12.0000 47.0000) (end 8.0000 47.0000) (width 0.6000) (layer "F.Cu") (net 7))
 (segment (start 8.0000 47.0000) (end 8.0000 44.0000) (width 0.6000) (layer "F.Cu") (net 7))
 (segment (start 8.0000 44.0000) (end 7.5000 44.0000) (width 0.6000) (layer "F.Cu") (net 7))
 (segment (start 7.5000 44.0000) (end 7.5000 41.5000) (width 0.6000) (layer "F.Cu") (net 7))
 (segment (start 7.5000 41.5000) (end 7.0000 41.5000) (width 0.6000) (layer "F.Cu") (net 7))
 (segment (start 7.0000 41.5000) (end 7.0000 39.0000) (width 0.6000) (layer "F.Cu") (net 7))
 (segment (start 31.0000 44.0000) (end 31.0000 42.0000) (width 0.6000) (layer "F.Cu") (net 7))
 (segment (start 31.0000 42.0000) (end 34.5000 42.0000) (width 0.6000) (layer "F.Cu") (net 7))
 (segment (start 34.5000 42.0000) (end 34.5000 41.5000) (width 0.6000) (layer "F.Cu") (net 7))
 (segment (start 34.5000 41.5000) (end 35.0000 41.5000) (width 0.6000) (layer "F.Cu") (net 7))
 (segment (start 35.0000 41.5000) (end 35.0000 40.0000) (width 0.6000) (layer "F.Cu") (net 7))
 (segment (start 35.0000 40.0000) (end 35.5000 40.0000) (width 0.6000) (layer "F.Cu") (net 7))
 (segment (start 35.5000 40.0000) (end 35.5000 39.0000) (width 0.6000) (layer "F.Cu") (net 7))
 (segment (start 35.5000 39.0000) (end 37.0000 39.0000) (width 0.6000) (layer "F.Cu") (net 7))
 (segment (start 37.0000 39.0000) (end 37.0000 38.5000) (width 0.6000) (layer "F.Cu") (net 7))
 (segment (start 37.0000 38.5000) (end 39.0000 38.5000) (width 0.6000) (layer "F.Cu") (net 7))
 (segment (start 39.0000 38.5000) (end 39.0000 38.0000) (width 0.6000) (layer "F.Cu") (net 7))
 (segment (start 39.0000 38.0000) (end 40.0000 38.0000) (width 0.6000) (layer "F.Cu") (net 7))
 (segment (start 40.0000 38.0000) (end 40.0000 37.5000) (width 0.6000) (layer "F.Cu") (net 7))
 (segment (start 40.0000 37.5000) (end 40.5000 37.5000) (width 0.6000) (layer "F.Cu") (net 7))
 (segment (start 40.5000 37.5000) (end 40.5000 37.0000) (width 0.6000) (layer "F.Cu") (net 7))
 (segment (start 40.5000 37.0000) (end 41.0000 37.0000) (width 0.6000) (layer "F.Cu") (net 7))
 (segment (start 41.0000 37.0000) (end 41.0000 33.5000) (width 0.6000) (layer "F.Cu") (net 7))
 (segment (start 41.0000 33.5000) (end 41.5000 33.5000) (width 0.6000) (layer "F.Cu") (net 7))
 (segment (start 41.5000 33.5000) (end 41.5000 33.0000) (width 0.6000) (layer "F.Cu") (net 7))
 (segment (start 41.5000 33.0000) (end 42.0000 33.0000) (width 0.6000) (layer "F.Cu") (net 7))
 (segment (start 42.0000 33.0000) (end 42.0000 32.5000) (width 0.6000) (layer "F.Cu") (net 7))
 (segment (start 42.0000 32.5000) (end 43.5000 32.5000) (width 0.6000) (layer "F.Cu") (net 7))
 (segment (start 43.5000 32.5000) (end 43.5000 29.5000) (width 0.6000) (layer "F.Cu") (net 7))
 (segment (start 43.5000 29.5000) (end 44.0000 29.5000) (width 0.6000) (layer "F.Cu") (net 7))
 (segment (start 44.0000 29.5000) (end 44.0000 26.0000) (width 0.6000) (layer "F.Cu") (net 7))
 (segment (start 44.0000 26.0000) (end 57.0000 26.0000) (width 0.6000) (layer "F.Cu") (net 7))
 (segment (start 57.0000 26.0000) (end 57.0000 25.5000) (width 0.6000) (layer "F.Cu") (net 7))
 (segment (start 57.0000 25.5000) (end 59.0000 25.5000) (width 0.6000) (layer "F.Cu") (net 7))
 (segment (start 59.0000 25.5000) (end 59.0000 7.0000) (width 0.6000) (layer "F.Cu") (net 7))
 (segment (start 59.0000 7.0000) (end 58.5000 7.0000) (width 0.6000) (layer "F.Cu") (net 7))
 (segment (start 58.5000 7.0000) (end 58.5000 6.5000) (width 0.6000) (layer "F.Cu") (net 7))
 (segment (start 58.5000 6.5000) (end 58.0000 6.5000) (width 0.6000) (layer "F.Cu") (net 7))
 (segment (start 58.0000 6.5000) (end 58.0000 6.0000) (width 0.6000) (layer "F.Cu") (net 7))
 (segment (start 58.0000 6.0000) (end 51.0000 6.0000) (width 0.6000) (layer "F.Cu") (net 7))
 (segment (start 51.0000 6.0000) (end 51.0000 6.5000) (width 0.6000) (layer "F.Cu") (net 7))
 (segment (start 51.0000 6.5000) (end 50.5000 6.5000) (width 0.6000) (layer "F.Cu") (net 7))
 (segment (start 50.5000 6.5000) (end 50.5000 7.0000) (width 0.6000) (layer "F.Cu") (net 7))
 (segment (start 50.5000 7.0000) (end 43.0000 7.0000) (width 0.6000) (layer "F.Cu") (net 7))
 (segment (start 43.0000 7.0000) (end 43.0000 7.5000) (width 0.6000) (layer "F.Cu") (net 7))
 (segment (start 43.0000 7.5000) (end 39.5000 7.5000) (width 0.6000) (layer "F.Cu") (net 7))
 (segment (start 39.5000 7.5000) (end 39.5000 8.5000) (width 0.6000) (layer "F.Cu") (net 7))
 (segment (start 39.5000 8.5000) (end 11.5000 8.5000) (width 0.6000) (layer "F.Cu") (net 7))
 (segment (start 11.5000 8.5000) (end 11.5000 9.5000) (width 0.6000) (layer "F.Cu") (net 7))
 (segment (start 61.0000 9.0000) (end 59.0000 9.0000) (width 0.6000) (layer "F.Cu") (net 7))
 (segment (start 59.0000 35.0000) (end 59.0000 25.5000) (width 0.6000) (layer "F.Cu") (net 7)))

